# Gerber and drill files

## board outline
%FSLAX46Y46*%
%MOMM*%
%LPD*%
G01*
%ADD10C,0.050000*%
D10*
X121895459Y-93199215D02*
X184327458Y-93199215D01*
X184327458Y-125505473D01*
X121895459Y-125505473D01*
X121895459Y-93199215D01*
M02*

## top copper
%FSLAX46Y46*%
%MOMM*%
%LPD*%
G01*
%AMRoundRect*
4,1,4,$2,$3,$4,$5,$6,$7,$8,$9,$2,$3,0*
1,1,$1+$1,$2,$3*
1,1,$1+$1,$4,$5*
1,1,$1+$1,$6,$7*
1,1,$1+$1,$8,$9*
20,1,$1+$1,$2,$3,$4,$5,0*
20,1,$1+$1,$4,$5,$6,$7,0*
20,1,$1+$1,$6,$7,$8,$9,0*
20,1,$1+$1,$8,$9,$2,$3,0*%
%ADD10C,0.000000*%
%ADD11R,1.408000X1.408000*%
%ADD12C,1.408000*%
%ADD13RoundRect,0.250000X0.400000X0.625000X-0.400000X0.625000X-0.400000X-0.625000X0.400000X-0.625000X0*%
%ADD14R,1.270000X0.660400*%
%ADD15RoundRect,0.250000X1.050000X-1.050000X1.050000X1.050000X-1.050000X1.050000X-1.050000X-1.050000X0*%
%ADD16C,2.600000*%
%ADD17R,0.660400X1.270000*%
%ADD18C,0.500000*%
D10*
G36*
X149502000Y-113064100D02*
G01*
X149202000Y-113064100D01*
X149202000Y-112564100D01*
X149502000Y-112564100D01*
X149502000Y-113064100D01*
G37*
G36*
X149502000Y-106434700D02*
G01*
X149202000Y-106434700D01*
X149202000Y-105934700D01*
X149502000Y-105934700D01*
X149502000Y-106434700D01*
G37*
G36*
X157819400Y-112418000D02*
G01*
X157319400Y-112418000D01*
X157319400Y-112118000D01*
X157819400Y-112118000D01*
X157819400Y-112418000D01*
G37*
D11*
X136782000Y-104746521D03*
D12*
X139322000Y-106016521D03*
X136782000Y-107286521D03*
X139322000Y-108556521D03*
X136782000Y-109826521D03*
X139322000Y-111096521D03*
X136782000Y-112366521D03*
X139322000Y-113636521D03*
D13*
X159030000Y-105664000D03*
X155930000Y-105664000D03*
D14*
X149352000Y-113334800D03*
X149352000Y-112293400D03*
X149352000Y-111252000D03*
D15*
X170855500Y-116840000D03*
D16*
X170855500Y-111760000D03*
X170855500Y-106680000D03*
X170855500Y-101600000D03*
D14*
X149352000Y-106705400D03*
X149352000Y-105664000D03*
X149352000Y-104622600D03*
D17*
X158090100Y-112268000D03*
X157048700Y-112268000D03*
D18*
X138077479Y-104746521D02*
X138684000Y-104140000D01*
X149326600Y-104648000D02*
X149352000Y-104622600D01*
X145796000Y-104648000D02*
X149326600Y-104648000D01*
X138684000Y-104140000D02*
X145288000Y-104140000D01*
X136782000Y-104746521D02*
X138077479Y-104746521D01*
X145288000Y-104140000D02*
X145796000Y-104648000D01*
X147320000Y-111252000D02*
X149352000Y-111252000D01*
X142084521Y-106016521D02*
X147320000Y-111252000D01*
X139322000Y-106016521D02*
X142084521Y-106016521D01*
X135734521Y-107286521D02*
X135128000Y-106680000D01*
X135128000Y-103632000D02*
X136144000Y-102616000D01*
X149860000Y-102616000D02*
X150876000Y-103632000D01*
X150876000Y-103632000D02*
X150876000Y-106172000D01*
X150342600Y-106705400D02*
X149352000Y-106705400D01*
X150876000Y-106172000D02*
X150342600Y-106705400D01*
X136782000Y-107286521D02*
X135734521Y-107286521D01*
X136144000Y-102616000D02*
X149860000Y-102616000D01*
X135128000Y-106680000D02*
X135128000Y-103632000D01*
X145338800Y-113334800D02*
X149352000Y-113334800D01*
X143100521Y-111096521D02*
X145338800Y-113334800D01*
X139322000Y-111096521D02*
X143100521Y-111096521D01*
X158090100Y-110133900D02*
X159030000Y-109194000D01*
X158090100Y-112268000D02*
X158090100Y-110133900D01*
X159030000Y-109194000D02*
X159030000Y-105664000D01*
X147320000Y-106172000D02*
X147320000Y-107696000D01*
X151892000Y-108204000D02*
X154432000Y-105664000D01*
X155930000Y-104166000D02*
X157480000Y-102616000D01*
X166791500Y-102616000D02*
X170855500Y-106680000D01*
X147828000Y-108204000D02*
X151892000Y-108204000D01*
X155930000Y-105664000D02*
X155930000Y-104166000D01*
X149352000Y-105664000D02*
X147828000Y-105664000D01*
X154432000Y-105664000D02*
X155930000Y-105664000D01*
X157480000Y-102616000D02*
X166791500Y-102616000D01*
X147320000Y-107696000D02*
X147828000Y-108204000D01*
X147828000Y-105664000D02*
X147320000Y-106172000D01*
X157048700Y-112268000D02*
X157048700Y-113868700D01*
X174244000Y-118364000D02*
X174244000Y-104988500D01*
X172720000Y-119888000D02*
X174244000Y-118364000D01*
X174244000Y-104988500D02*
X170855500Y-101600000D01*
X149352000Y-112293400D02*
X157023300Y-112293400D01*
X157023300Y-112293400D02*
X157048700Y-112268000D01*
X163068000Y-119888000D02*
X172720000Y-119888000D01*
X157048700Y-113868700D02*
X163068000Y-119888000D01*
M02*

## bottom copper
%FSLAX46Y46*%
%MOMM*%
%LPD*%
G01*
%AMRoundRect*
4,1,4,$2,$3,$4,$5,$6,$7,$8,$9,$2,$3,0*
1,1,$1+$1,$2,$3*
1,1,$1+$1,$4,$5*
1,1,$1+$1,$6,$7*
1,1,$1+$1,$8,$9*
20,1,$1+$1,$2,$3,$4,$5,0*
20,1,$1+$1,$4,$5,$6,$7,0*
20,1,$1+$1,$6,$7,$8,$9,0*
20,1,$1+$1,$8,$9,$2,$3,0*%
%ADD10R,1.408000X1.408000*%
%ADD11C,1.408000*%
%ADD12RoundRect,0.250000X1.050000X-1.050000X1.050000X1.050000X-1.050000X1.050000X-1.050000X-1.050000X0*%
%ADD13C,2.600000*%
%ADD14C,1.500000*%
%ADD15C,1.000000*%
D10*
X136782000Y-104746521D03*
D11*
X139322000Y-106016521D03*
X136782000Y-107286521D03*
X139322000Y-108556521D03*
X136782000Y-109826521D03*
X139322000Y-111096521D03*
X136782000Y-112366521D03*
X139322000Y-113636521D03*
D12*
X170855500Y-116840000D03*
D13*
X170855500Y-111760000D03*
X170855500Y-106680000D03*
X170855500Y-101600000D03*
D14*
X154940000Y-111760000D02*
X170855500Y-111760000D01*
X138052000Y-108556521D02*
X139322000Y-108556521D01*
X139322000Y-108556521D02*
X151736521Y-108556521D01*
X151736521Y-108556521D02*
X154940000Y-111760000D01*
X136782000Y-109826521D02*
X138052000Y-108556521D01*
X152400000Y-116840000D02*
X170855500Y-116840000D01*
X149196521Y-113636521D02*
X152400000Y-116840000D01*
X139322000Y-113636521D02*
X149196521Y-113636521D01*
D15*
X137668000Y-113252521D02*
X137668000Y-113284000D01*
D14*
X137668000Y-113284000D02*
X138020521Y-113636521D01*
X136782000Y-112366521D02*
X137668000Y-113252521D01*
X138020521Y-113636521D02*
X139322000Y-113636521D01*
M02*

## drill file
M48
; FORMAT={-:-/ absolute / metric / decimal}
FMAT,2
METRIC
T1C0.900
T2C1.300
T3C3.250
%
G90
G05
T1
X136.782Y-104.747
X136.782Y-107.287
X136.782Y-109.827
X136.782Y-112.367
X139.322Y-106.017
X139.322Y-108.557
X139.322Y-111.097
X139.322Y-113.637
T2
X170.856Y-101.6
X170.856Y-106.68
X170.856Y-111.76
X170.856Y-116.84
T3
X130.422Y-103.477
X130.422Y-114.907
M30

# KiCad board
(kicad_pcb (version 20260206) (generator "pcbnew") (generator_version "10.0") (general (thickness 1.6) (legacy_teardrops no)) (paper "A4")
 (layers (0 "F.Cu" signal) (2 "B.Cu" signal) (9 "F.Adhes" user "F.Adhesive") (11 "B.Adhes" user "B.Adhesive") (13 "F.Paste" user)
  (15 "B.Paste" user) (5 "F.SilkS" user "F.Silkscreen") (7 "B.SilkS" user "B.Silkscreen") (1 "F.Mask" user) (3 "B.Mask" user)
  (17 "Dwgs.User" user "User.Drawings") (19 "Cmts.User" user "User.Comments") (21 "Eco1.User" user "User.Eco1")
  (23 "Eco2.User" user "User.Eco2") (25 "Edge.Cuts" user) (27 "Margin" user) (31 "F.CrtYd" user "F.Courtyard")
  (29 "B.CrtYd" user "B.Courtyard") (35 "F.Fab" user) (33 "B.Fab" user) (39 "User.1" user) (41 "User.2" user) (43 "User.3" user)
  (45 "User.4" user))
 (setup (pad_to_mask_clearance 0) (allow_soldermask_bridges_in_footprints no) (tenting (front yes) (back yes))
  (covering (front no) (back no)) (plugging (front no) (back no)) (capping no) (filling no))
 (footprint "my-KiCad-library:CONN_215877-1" (layer "F.Cu") (at 130.422 109.191521 -90)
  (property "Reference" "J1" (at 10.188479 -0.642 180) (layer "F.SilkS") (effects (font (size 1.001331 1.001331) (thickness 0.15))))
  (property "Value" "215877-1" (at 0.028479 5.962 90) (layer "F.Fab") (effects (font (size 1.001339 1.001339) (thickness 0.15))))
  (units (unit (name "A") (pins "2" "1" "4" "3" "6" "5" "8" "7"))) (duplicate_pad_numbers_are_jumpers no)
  (pad "" np_thru_hole circle (at -5.715 0 270) (size 3.25 3.25) (drill 3.25) (layers "*.Cu" "*.Mask"))
  (pad "" np_thru_hole circle (at 5.715 0 270) (size 3.25 3.25) (drill 3.25) (layers "*.Cu" "*.Mask"))
  (pad "1" thru_hole rect (at -4.445 -6.36 270) (size 1.408 1.408) (drill 0.9) (layers "*.Cu" "*.Mask") (remove_unused_layers no)
   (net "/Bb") (solder_mask_margin 0.102))
  (pad "2" thru_hole circle (at -3.175 -8.9 270) (size 1.408 1.408) (drill 0.9) (layers "*.Cu" "*.Mask") (remove_unused_layers no)
   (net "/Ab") (solder_mask_margin 0.102))
  (pad "3" thru_hole circle (at -1.905 -6.36 270) (size 1.408 1.408) (drill 0.9) (layers "*.Cu" "*.Mask") (remove_unused_layers no)
   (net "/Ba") (solder_mask_margin 0.102))
  (pad "4" thru_hole circle (at -0.635 -8.9 270) (size 1.408 1.408) (drill 0.9) (layers "*.Cu" "*.Mask") (remove_unused_layers no)
   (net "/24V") (solder_mask_margin 0.102))
  (pad "5" thru_hole circle (at 0.635 -6.36 270) (size 1.408 1.408) (drill 0.9) (layers "*.Cu" "*.Mask") (remove_unused_layers no)
   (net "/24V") (solder_mask_margin 0.102))
  (pad "6" thru_hole circle (at 1.905 -8.9 270) (size 1.408 1.408) (drill 0.9) (layers "*.Cu" "*.Mask") (remove_unused_layers no)
   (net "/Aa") (solder_mask_margin 0.102))
  (pad "7" thru_hole circle (at 3.175 -6.36 270) (size 1.408 1.408) (drill 0.9) (layers "*.Cu" "*.Mask") (remove_unused_layers no)
   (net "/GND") (solder_mask_margin 0.102))
  (pad "8" thru_hole circle (at 4.445 -8.9 270) (size 1.408 1.408) (drill 0.9) (layers "*.Cu" "*.Mask") (remove_unused_layers no)
   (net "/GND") (solder_mask_margin 0.102)))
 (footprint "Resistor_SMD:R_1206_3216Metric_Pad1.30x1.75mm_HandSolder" (layer "F.Cu") (at 157.48 105.664 180)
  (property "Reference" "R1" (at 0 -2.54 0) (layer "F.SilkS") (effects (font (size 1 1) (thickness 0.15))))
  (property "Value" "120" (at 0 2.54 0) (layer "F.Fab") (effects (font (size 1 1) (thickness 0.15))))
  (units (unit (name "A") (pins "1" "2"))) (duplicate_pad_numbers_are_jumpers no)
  (pad "1" smd roundrect (at -1.55 0 180) (size 1.3 1.75) (layers "F.Cu" "F.Mask" "F.Paste") (roundrect_rratio 0.192308) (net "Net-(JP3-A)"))
  (pad "2" smd roundrect (at 1.55 0 180) (size 1.3 1.75) (layers "F.Cu" "F.Mask" "F.Paste") (roundrect_rratio 0.192308) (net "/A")))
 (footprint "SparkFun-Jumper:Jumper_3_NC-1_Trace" (layer "F.Cu") (at 149.352 112.2934 90)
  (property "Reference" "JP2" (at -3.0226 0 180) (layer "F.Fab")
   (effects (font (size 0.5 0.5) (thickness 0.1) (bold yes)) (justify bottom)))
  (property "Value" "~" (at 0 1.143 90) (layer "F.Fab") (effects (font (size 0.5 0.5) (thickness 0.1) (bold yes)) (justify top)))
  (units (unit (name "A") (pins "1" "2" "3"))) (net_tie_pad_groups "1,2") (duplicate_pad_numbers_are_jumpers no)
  (fp_poly
   (pts (xy -0.7707 -0.15) (xy -0.2707 -0.15) (xy -0.2707 0.15) (xy -0.7707 0.15)) (stroke (width 0) (type solid)) (fill yes) (layer "F.Cu"))
  (pad "1" smd rect (at -1.0414 0 90) (size 0.6604 1.27) (layers "F.Cu" "F.Mask") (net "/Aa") (thermal_bridge_angle 0))
  (pad "2" smd rect (at 0 0 90) (size 0.6604 1.27) (layers "F.Cu" "F.Mask") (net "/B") (thermal_bridge_angle 0))
  (pad "3" smd rect (at 1.0414 0 270) (size 0.6604 1.27) (layers "F.Cu" "F.Mask") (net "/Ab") (thermal_bridge_angle 0)))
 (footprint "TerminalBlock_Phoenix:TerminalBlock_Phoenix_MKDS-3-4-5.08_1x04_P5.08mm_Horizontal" (layer "F.Cu") (at 170.8555 116.84 90)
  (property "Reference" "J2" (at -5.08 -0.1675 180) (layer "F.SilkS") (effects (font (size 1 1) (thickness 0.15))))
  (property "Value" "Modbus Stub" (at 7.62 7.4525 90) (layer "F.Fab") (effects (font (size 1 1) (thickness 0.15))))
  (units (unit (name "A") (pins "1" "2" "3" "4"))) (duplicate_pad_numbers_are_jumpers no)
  (pad "1" thru_hole roundrect (at 0 0 90) (size 2.6 2.6) (drill 1.3) (layers "*.Cu" "*.Mask") (remove_unused_layers no)
   (roundrect_rratio 0.096154) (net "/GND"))
  (pad "2" thru_hole circle (at 5.08 0 90) (size 2.6 2.6) (drill 1.3) (layers "*.Cu" "*.Mask") (remove_unused_layers no) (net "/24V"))
  (pad "3" thru_hole circle (at 10.16 0 90) (size 2.6 2.6) (drill 1.3) (layers "*.Cu" "*.Mask") (remove_unused_layers no) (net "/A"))
  (pad "4" thru_hole circle (at 15.24 0 90) (size 2.6 2.6) (drill 1.3) (layers "*.Cu" "*.Mask") (remove_unused_layers no) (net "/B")))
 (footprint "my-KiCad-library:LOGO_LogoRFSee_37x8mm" (layer "F.Cu") (at 152.4 120.904)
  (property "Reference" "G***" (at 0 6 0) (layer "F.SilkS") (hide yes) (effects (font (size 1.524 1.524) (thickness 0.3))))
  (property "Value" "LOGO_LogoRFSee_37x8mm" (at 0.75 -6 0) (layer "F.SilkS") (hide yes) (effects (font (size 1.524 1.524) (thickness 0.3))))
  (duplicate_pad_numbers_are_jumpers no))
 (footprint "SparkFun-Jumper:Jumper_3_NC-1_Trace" (layer "F.Cu") (at 149.352 105.664 90)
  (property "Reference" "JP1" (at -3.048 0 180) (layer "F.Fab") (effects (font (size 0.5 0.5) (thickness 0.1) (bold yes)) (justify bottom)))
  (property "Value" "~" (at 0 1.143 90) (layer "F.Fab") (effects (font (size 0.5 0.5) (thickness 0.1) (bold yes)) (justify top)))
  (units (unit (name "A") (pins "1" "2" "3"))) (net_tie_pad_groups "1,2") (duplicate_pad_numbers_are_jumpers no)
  (fp_poly
   (pts (xy -0.7707 -0.15) (xy -0.2707 -0.15) (xy -0.2707 0.15) (xy -0.7707 0.15)) (stroke (width 0) (type solid)) (fill yes) (layer "F.Cu"))
  (pad "1" smd rect (at -1.0414 0 90) (size 0.6604 1.27) (layers "F.Cu" "F.Mask") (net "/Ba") (thermal_bridge_angle 0))
  (pad "2" smd rect (at 0 0 90) (size 0.6604 1.27) (layers "F.Cu" "F.Mask") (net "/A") (thermal_bridge_angle 0))
  (pad "3" smd rect (at 1.0414 0 270) (size 0.6604 1.27) (layers "F.Cu" "F.Mask") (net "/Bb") (thermal_bridge_angle 0)))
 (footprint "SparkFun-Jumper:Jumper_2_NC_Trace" (layer "F.Cu") (at 157.5694 112.268 180)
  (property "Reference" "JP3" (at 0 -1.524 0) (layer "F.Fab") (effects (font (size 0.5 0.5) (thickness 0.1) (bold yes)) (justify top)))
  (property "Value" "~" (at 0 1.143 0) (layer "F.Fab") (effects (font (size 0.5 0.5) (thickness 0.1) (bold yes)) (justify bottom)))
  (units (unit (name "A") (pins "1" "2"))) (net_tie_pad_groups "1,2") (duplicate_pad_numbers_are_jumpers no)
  (fp_poly (pts (xy -0.25 -0.15) (xy 0.25 -0.15) (xy 0.25 0.15) (xy -0.25 0.15)) (stroke (width 0) (type solid)) (fill yes) (layer "F.Cu"))
  (pad "1" smd rect (at -0.5207 0 180) (size 0.6604 1.27) (layers "F.Cu" "F.Mask") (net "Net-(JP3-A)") (thermal_bridge_angle 0))
  (pad "2" smd rect (at 0.5207 0 180) (size 0.6604 1.27) (layers "F.Cu" "F.Mask") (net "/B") (thermal_bridge_angle 0)))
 (gr_rect (start 121.895459 93.199215) (end 184.327458 125.505473) (stroke (width 0.05) (type solid)) (fill no) (layer "Edge.Cuts"))
 (segment (start 138.077479 104.746521) (end 138.684 104.14) (width 0.5) (layer "F.Cu") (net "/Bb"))
 (segment (start 149.3266 104.648) (end 149.352 104.6226) (width 0.5) (layer "F.Cu") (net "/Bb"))
 (segment (start 145.796 104.648) (end 149.3266 104.648) (width 0.5) (layer "F.Cu") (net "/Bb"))
 (segment (start 138.684 104.14) (end 145.288 104.14) (width 0.5) (layer "F.Cu") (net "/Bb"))
 (segment (start 136.782 104.746521) (end 138.077479 104.746521) (width 0.5) (layer "F.Cu") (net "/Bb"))
 (segment (start 145.288 104.14) (end 145.796 104.648) (width 0.5) (layer "F.Cu") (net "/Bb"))
 (segment (start 147.32 111.252) (end 149.352 111.252) (width 0.5) (layer "F.Cu") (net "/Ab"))
 (segment (start 142.084521 106.016521) (end 147.32 111.252) (width 0.5) (layer "F.Cu") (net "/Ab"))
 (segment (start 139.322 106.016521) (end 142.084521 106.016521) (width 0.5) (layer "F.Cu") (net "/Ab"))
 (segment (start 135.734521 107.286521) (end 135.128 106.68) (width 0.5) (layer "F.Cu") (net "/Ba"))
 (segment (start 135.128 103.632) (end 136.144 102.616) (width 0.5) (layer "F.Cu") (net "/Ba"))
 (segment (start 149.86 102.616) (end 150.876 103.632) (width 0.5) (layer "F.Cu") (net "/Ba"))
 (segment (start 150.876 103.632) (end 150.876 106.172) (width 0.5) (layer "F.Cu") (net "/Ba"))
 (segment (start 150.3426 106.7054) (end 149.352 106.7054) (width 0.5) (layer "F.Cu") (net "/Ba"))
 (segment (start 150.876 106.172) (end 150.3426 106.7054) (width 0.5) (layer "F.Cu") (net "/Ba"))
 (segment (start 136.782 107.286521) (end 135.734521 107.286521) (width 0.5) (layer "F.Cu") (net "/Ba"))
 (segment (start 136.144 102.616) (end 149.86 102.616) (width 0.5) (layer "F.Cu") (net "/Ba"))
 (segment (start 135.128 106.68) (end 135.128 103.632) (width 0.5) (layer "F.Cu") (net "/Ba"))
 (segment (start 154.94 111.76) (end 170.8555 111.76) (width 1.5) (layer "B.Cu") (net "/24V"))
 (segment (start 138.052 108.556521) (end 139.322 108.556521) (width 1.5) (layer "B.Cu") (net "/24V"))
 (segment (start 139.322 108.556521) (end 151.736521 108.556521) (width 1.5) (layer "B.Cu") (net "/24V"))
 (segment (start 151.736521 108.556521) (end 154.94 111.76) (width 1.5) (layer "B.Cu") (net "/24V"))
 (segment (start 136.782 109.826521) (end 138.052 108.556521) (width 1.5) (layer "B.Cu") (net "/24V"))
 (segment (start 145.3388 113.3348) (end 149.352 113.3348) (width 0.5) (layer "F.Cu") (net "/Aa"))
 (segment (start 143.100521 111.096521) (end 145.3388 113.3348) (width 0.5) (layer "F.Cu") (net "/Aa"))
 (segment (start 139.322 111.096521) (end 143.100521 111.096521) (width 0.5) (layer "F.Cu") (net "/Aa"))
 (segment (start 152.4 116.84) (end 170.8555 116.84) (width 1.5) (layer "B.Cu") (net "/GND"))
 (segment (start 149.196521 113.636521) (end 152.4 116.84) (width 1.5) (layer "B.Cu") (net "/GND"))
 (segment (start 139.322 113.636521) (end 149.196521 113.636521) (width 1.5) (layer "B.Cu") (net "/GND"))
 (segment (start 137.668 113.252521) (end 137.668 113.284) (width 1) (layer "B.Cu") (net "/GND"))
 (segment (start 137.668 113.284) (end 138.020521 113.636521) (width 1.5) (layer "B.Cu") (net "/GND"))
 (segment (start 136.782 112.366521) (end 137.668 113.252521) (width 1.5) (layer "B.Cu") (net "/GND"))
 (segment (start 138.020521 113.636521) (end 139.322 113.636521) (width 1.5) (layer "B.Cu") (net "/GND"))
 (segment (start 158.0901 110.1339) (end 159.03 109.194) (width 0.5) (layer "F.Cu") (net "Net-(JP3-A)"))
 (segment (start 158.0901 112.268) (end 158.0901 110.1339) (width 0.5) (layer "F.Cu") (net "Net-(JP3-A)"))
 (segment (start 159.03 109.194) (end 159.03 105.664) (width 0.5) (layer "F.Cu") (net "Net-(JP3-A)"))
 (segment (start 147.32 106.172) (end 147.32 107.696) (width 0.5) (layer "F.Cu") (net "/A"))
 (segment (start 151.892 108.204) (end 154.432 105.664) (width 0.5) (layer "F.Cu") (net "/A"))
 (segment (start 155.93 104.166) (end 157.48 102.616) (width 0.5) (layer "F.Cu") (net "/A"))
 (segment (start 166.7915 102.616) (end 170.8555 106.68) (width 0.5) (layer "F.Cu") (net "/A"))
 (segment (start 147.828 108.204) (end 151.892 108.204) (width 0.5) (layer "F.Cu") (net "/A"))
 (segment (start 155.93 105.664) (end 155.93 104.166) (width 0.5) (layer "F.Cu") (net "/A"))
 (segment (start 149.352 105.664) (end 147.828 105.664) (width 0.5) (layer "F.Cu") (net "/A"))
 (segment (start 154.432 105.664) (end 155.93 105.664) (width 0.5) (layer "F.Cu") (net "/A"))
 (segment (start 157.48 102.616) (end 166.7915 102.616) (width 0.5) (layer "F.Cu") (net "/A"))
 (segment (start 147.32 107.696) (end 147.828 108.204) (width 0.5) (layer "F.Cu") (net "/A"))
 (segment (start 147.828 105.664) (end 147.32 106.172) (width 0.5) (layer "F.Cu") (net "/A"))
 (segment (start 157.0487 112.268) (end 157.0487 113.8687) (width 0.5) (layer "F.Cu") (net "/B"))
 (segment (start 174.244 118.364) (end 174.244 104.9885) (width 0.5) (layer "F.Cu") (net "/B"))
 (segment (start 172.72 119.888) (end 174.244 118.364) (width 0.5) (layer "F.Cu") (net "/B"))
 (segment (start 174.244 104.9885) (end 170.8555 101.6) (width 0.5) (layer "F.Cu") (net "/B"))
 (segment (start 149.352 112.2934) (end 157.0233 112.2934) (width 0.5) (layer "F.Cu") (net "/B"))
 (segment (start 157.0233 112.2934) (end 157.0487 112.268) (width 0.5) (layer "F.Cu") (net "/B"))
 (segment (start 163.068 119.888) (end 172.72 119.888) (width 0.5) (layer "F.Cu") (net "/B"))
 (segment (start 157.0487 113.8687) (end 163.068 119.888) (width 0.5) (layer "F.Cu") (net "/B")))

